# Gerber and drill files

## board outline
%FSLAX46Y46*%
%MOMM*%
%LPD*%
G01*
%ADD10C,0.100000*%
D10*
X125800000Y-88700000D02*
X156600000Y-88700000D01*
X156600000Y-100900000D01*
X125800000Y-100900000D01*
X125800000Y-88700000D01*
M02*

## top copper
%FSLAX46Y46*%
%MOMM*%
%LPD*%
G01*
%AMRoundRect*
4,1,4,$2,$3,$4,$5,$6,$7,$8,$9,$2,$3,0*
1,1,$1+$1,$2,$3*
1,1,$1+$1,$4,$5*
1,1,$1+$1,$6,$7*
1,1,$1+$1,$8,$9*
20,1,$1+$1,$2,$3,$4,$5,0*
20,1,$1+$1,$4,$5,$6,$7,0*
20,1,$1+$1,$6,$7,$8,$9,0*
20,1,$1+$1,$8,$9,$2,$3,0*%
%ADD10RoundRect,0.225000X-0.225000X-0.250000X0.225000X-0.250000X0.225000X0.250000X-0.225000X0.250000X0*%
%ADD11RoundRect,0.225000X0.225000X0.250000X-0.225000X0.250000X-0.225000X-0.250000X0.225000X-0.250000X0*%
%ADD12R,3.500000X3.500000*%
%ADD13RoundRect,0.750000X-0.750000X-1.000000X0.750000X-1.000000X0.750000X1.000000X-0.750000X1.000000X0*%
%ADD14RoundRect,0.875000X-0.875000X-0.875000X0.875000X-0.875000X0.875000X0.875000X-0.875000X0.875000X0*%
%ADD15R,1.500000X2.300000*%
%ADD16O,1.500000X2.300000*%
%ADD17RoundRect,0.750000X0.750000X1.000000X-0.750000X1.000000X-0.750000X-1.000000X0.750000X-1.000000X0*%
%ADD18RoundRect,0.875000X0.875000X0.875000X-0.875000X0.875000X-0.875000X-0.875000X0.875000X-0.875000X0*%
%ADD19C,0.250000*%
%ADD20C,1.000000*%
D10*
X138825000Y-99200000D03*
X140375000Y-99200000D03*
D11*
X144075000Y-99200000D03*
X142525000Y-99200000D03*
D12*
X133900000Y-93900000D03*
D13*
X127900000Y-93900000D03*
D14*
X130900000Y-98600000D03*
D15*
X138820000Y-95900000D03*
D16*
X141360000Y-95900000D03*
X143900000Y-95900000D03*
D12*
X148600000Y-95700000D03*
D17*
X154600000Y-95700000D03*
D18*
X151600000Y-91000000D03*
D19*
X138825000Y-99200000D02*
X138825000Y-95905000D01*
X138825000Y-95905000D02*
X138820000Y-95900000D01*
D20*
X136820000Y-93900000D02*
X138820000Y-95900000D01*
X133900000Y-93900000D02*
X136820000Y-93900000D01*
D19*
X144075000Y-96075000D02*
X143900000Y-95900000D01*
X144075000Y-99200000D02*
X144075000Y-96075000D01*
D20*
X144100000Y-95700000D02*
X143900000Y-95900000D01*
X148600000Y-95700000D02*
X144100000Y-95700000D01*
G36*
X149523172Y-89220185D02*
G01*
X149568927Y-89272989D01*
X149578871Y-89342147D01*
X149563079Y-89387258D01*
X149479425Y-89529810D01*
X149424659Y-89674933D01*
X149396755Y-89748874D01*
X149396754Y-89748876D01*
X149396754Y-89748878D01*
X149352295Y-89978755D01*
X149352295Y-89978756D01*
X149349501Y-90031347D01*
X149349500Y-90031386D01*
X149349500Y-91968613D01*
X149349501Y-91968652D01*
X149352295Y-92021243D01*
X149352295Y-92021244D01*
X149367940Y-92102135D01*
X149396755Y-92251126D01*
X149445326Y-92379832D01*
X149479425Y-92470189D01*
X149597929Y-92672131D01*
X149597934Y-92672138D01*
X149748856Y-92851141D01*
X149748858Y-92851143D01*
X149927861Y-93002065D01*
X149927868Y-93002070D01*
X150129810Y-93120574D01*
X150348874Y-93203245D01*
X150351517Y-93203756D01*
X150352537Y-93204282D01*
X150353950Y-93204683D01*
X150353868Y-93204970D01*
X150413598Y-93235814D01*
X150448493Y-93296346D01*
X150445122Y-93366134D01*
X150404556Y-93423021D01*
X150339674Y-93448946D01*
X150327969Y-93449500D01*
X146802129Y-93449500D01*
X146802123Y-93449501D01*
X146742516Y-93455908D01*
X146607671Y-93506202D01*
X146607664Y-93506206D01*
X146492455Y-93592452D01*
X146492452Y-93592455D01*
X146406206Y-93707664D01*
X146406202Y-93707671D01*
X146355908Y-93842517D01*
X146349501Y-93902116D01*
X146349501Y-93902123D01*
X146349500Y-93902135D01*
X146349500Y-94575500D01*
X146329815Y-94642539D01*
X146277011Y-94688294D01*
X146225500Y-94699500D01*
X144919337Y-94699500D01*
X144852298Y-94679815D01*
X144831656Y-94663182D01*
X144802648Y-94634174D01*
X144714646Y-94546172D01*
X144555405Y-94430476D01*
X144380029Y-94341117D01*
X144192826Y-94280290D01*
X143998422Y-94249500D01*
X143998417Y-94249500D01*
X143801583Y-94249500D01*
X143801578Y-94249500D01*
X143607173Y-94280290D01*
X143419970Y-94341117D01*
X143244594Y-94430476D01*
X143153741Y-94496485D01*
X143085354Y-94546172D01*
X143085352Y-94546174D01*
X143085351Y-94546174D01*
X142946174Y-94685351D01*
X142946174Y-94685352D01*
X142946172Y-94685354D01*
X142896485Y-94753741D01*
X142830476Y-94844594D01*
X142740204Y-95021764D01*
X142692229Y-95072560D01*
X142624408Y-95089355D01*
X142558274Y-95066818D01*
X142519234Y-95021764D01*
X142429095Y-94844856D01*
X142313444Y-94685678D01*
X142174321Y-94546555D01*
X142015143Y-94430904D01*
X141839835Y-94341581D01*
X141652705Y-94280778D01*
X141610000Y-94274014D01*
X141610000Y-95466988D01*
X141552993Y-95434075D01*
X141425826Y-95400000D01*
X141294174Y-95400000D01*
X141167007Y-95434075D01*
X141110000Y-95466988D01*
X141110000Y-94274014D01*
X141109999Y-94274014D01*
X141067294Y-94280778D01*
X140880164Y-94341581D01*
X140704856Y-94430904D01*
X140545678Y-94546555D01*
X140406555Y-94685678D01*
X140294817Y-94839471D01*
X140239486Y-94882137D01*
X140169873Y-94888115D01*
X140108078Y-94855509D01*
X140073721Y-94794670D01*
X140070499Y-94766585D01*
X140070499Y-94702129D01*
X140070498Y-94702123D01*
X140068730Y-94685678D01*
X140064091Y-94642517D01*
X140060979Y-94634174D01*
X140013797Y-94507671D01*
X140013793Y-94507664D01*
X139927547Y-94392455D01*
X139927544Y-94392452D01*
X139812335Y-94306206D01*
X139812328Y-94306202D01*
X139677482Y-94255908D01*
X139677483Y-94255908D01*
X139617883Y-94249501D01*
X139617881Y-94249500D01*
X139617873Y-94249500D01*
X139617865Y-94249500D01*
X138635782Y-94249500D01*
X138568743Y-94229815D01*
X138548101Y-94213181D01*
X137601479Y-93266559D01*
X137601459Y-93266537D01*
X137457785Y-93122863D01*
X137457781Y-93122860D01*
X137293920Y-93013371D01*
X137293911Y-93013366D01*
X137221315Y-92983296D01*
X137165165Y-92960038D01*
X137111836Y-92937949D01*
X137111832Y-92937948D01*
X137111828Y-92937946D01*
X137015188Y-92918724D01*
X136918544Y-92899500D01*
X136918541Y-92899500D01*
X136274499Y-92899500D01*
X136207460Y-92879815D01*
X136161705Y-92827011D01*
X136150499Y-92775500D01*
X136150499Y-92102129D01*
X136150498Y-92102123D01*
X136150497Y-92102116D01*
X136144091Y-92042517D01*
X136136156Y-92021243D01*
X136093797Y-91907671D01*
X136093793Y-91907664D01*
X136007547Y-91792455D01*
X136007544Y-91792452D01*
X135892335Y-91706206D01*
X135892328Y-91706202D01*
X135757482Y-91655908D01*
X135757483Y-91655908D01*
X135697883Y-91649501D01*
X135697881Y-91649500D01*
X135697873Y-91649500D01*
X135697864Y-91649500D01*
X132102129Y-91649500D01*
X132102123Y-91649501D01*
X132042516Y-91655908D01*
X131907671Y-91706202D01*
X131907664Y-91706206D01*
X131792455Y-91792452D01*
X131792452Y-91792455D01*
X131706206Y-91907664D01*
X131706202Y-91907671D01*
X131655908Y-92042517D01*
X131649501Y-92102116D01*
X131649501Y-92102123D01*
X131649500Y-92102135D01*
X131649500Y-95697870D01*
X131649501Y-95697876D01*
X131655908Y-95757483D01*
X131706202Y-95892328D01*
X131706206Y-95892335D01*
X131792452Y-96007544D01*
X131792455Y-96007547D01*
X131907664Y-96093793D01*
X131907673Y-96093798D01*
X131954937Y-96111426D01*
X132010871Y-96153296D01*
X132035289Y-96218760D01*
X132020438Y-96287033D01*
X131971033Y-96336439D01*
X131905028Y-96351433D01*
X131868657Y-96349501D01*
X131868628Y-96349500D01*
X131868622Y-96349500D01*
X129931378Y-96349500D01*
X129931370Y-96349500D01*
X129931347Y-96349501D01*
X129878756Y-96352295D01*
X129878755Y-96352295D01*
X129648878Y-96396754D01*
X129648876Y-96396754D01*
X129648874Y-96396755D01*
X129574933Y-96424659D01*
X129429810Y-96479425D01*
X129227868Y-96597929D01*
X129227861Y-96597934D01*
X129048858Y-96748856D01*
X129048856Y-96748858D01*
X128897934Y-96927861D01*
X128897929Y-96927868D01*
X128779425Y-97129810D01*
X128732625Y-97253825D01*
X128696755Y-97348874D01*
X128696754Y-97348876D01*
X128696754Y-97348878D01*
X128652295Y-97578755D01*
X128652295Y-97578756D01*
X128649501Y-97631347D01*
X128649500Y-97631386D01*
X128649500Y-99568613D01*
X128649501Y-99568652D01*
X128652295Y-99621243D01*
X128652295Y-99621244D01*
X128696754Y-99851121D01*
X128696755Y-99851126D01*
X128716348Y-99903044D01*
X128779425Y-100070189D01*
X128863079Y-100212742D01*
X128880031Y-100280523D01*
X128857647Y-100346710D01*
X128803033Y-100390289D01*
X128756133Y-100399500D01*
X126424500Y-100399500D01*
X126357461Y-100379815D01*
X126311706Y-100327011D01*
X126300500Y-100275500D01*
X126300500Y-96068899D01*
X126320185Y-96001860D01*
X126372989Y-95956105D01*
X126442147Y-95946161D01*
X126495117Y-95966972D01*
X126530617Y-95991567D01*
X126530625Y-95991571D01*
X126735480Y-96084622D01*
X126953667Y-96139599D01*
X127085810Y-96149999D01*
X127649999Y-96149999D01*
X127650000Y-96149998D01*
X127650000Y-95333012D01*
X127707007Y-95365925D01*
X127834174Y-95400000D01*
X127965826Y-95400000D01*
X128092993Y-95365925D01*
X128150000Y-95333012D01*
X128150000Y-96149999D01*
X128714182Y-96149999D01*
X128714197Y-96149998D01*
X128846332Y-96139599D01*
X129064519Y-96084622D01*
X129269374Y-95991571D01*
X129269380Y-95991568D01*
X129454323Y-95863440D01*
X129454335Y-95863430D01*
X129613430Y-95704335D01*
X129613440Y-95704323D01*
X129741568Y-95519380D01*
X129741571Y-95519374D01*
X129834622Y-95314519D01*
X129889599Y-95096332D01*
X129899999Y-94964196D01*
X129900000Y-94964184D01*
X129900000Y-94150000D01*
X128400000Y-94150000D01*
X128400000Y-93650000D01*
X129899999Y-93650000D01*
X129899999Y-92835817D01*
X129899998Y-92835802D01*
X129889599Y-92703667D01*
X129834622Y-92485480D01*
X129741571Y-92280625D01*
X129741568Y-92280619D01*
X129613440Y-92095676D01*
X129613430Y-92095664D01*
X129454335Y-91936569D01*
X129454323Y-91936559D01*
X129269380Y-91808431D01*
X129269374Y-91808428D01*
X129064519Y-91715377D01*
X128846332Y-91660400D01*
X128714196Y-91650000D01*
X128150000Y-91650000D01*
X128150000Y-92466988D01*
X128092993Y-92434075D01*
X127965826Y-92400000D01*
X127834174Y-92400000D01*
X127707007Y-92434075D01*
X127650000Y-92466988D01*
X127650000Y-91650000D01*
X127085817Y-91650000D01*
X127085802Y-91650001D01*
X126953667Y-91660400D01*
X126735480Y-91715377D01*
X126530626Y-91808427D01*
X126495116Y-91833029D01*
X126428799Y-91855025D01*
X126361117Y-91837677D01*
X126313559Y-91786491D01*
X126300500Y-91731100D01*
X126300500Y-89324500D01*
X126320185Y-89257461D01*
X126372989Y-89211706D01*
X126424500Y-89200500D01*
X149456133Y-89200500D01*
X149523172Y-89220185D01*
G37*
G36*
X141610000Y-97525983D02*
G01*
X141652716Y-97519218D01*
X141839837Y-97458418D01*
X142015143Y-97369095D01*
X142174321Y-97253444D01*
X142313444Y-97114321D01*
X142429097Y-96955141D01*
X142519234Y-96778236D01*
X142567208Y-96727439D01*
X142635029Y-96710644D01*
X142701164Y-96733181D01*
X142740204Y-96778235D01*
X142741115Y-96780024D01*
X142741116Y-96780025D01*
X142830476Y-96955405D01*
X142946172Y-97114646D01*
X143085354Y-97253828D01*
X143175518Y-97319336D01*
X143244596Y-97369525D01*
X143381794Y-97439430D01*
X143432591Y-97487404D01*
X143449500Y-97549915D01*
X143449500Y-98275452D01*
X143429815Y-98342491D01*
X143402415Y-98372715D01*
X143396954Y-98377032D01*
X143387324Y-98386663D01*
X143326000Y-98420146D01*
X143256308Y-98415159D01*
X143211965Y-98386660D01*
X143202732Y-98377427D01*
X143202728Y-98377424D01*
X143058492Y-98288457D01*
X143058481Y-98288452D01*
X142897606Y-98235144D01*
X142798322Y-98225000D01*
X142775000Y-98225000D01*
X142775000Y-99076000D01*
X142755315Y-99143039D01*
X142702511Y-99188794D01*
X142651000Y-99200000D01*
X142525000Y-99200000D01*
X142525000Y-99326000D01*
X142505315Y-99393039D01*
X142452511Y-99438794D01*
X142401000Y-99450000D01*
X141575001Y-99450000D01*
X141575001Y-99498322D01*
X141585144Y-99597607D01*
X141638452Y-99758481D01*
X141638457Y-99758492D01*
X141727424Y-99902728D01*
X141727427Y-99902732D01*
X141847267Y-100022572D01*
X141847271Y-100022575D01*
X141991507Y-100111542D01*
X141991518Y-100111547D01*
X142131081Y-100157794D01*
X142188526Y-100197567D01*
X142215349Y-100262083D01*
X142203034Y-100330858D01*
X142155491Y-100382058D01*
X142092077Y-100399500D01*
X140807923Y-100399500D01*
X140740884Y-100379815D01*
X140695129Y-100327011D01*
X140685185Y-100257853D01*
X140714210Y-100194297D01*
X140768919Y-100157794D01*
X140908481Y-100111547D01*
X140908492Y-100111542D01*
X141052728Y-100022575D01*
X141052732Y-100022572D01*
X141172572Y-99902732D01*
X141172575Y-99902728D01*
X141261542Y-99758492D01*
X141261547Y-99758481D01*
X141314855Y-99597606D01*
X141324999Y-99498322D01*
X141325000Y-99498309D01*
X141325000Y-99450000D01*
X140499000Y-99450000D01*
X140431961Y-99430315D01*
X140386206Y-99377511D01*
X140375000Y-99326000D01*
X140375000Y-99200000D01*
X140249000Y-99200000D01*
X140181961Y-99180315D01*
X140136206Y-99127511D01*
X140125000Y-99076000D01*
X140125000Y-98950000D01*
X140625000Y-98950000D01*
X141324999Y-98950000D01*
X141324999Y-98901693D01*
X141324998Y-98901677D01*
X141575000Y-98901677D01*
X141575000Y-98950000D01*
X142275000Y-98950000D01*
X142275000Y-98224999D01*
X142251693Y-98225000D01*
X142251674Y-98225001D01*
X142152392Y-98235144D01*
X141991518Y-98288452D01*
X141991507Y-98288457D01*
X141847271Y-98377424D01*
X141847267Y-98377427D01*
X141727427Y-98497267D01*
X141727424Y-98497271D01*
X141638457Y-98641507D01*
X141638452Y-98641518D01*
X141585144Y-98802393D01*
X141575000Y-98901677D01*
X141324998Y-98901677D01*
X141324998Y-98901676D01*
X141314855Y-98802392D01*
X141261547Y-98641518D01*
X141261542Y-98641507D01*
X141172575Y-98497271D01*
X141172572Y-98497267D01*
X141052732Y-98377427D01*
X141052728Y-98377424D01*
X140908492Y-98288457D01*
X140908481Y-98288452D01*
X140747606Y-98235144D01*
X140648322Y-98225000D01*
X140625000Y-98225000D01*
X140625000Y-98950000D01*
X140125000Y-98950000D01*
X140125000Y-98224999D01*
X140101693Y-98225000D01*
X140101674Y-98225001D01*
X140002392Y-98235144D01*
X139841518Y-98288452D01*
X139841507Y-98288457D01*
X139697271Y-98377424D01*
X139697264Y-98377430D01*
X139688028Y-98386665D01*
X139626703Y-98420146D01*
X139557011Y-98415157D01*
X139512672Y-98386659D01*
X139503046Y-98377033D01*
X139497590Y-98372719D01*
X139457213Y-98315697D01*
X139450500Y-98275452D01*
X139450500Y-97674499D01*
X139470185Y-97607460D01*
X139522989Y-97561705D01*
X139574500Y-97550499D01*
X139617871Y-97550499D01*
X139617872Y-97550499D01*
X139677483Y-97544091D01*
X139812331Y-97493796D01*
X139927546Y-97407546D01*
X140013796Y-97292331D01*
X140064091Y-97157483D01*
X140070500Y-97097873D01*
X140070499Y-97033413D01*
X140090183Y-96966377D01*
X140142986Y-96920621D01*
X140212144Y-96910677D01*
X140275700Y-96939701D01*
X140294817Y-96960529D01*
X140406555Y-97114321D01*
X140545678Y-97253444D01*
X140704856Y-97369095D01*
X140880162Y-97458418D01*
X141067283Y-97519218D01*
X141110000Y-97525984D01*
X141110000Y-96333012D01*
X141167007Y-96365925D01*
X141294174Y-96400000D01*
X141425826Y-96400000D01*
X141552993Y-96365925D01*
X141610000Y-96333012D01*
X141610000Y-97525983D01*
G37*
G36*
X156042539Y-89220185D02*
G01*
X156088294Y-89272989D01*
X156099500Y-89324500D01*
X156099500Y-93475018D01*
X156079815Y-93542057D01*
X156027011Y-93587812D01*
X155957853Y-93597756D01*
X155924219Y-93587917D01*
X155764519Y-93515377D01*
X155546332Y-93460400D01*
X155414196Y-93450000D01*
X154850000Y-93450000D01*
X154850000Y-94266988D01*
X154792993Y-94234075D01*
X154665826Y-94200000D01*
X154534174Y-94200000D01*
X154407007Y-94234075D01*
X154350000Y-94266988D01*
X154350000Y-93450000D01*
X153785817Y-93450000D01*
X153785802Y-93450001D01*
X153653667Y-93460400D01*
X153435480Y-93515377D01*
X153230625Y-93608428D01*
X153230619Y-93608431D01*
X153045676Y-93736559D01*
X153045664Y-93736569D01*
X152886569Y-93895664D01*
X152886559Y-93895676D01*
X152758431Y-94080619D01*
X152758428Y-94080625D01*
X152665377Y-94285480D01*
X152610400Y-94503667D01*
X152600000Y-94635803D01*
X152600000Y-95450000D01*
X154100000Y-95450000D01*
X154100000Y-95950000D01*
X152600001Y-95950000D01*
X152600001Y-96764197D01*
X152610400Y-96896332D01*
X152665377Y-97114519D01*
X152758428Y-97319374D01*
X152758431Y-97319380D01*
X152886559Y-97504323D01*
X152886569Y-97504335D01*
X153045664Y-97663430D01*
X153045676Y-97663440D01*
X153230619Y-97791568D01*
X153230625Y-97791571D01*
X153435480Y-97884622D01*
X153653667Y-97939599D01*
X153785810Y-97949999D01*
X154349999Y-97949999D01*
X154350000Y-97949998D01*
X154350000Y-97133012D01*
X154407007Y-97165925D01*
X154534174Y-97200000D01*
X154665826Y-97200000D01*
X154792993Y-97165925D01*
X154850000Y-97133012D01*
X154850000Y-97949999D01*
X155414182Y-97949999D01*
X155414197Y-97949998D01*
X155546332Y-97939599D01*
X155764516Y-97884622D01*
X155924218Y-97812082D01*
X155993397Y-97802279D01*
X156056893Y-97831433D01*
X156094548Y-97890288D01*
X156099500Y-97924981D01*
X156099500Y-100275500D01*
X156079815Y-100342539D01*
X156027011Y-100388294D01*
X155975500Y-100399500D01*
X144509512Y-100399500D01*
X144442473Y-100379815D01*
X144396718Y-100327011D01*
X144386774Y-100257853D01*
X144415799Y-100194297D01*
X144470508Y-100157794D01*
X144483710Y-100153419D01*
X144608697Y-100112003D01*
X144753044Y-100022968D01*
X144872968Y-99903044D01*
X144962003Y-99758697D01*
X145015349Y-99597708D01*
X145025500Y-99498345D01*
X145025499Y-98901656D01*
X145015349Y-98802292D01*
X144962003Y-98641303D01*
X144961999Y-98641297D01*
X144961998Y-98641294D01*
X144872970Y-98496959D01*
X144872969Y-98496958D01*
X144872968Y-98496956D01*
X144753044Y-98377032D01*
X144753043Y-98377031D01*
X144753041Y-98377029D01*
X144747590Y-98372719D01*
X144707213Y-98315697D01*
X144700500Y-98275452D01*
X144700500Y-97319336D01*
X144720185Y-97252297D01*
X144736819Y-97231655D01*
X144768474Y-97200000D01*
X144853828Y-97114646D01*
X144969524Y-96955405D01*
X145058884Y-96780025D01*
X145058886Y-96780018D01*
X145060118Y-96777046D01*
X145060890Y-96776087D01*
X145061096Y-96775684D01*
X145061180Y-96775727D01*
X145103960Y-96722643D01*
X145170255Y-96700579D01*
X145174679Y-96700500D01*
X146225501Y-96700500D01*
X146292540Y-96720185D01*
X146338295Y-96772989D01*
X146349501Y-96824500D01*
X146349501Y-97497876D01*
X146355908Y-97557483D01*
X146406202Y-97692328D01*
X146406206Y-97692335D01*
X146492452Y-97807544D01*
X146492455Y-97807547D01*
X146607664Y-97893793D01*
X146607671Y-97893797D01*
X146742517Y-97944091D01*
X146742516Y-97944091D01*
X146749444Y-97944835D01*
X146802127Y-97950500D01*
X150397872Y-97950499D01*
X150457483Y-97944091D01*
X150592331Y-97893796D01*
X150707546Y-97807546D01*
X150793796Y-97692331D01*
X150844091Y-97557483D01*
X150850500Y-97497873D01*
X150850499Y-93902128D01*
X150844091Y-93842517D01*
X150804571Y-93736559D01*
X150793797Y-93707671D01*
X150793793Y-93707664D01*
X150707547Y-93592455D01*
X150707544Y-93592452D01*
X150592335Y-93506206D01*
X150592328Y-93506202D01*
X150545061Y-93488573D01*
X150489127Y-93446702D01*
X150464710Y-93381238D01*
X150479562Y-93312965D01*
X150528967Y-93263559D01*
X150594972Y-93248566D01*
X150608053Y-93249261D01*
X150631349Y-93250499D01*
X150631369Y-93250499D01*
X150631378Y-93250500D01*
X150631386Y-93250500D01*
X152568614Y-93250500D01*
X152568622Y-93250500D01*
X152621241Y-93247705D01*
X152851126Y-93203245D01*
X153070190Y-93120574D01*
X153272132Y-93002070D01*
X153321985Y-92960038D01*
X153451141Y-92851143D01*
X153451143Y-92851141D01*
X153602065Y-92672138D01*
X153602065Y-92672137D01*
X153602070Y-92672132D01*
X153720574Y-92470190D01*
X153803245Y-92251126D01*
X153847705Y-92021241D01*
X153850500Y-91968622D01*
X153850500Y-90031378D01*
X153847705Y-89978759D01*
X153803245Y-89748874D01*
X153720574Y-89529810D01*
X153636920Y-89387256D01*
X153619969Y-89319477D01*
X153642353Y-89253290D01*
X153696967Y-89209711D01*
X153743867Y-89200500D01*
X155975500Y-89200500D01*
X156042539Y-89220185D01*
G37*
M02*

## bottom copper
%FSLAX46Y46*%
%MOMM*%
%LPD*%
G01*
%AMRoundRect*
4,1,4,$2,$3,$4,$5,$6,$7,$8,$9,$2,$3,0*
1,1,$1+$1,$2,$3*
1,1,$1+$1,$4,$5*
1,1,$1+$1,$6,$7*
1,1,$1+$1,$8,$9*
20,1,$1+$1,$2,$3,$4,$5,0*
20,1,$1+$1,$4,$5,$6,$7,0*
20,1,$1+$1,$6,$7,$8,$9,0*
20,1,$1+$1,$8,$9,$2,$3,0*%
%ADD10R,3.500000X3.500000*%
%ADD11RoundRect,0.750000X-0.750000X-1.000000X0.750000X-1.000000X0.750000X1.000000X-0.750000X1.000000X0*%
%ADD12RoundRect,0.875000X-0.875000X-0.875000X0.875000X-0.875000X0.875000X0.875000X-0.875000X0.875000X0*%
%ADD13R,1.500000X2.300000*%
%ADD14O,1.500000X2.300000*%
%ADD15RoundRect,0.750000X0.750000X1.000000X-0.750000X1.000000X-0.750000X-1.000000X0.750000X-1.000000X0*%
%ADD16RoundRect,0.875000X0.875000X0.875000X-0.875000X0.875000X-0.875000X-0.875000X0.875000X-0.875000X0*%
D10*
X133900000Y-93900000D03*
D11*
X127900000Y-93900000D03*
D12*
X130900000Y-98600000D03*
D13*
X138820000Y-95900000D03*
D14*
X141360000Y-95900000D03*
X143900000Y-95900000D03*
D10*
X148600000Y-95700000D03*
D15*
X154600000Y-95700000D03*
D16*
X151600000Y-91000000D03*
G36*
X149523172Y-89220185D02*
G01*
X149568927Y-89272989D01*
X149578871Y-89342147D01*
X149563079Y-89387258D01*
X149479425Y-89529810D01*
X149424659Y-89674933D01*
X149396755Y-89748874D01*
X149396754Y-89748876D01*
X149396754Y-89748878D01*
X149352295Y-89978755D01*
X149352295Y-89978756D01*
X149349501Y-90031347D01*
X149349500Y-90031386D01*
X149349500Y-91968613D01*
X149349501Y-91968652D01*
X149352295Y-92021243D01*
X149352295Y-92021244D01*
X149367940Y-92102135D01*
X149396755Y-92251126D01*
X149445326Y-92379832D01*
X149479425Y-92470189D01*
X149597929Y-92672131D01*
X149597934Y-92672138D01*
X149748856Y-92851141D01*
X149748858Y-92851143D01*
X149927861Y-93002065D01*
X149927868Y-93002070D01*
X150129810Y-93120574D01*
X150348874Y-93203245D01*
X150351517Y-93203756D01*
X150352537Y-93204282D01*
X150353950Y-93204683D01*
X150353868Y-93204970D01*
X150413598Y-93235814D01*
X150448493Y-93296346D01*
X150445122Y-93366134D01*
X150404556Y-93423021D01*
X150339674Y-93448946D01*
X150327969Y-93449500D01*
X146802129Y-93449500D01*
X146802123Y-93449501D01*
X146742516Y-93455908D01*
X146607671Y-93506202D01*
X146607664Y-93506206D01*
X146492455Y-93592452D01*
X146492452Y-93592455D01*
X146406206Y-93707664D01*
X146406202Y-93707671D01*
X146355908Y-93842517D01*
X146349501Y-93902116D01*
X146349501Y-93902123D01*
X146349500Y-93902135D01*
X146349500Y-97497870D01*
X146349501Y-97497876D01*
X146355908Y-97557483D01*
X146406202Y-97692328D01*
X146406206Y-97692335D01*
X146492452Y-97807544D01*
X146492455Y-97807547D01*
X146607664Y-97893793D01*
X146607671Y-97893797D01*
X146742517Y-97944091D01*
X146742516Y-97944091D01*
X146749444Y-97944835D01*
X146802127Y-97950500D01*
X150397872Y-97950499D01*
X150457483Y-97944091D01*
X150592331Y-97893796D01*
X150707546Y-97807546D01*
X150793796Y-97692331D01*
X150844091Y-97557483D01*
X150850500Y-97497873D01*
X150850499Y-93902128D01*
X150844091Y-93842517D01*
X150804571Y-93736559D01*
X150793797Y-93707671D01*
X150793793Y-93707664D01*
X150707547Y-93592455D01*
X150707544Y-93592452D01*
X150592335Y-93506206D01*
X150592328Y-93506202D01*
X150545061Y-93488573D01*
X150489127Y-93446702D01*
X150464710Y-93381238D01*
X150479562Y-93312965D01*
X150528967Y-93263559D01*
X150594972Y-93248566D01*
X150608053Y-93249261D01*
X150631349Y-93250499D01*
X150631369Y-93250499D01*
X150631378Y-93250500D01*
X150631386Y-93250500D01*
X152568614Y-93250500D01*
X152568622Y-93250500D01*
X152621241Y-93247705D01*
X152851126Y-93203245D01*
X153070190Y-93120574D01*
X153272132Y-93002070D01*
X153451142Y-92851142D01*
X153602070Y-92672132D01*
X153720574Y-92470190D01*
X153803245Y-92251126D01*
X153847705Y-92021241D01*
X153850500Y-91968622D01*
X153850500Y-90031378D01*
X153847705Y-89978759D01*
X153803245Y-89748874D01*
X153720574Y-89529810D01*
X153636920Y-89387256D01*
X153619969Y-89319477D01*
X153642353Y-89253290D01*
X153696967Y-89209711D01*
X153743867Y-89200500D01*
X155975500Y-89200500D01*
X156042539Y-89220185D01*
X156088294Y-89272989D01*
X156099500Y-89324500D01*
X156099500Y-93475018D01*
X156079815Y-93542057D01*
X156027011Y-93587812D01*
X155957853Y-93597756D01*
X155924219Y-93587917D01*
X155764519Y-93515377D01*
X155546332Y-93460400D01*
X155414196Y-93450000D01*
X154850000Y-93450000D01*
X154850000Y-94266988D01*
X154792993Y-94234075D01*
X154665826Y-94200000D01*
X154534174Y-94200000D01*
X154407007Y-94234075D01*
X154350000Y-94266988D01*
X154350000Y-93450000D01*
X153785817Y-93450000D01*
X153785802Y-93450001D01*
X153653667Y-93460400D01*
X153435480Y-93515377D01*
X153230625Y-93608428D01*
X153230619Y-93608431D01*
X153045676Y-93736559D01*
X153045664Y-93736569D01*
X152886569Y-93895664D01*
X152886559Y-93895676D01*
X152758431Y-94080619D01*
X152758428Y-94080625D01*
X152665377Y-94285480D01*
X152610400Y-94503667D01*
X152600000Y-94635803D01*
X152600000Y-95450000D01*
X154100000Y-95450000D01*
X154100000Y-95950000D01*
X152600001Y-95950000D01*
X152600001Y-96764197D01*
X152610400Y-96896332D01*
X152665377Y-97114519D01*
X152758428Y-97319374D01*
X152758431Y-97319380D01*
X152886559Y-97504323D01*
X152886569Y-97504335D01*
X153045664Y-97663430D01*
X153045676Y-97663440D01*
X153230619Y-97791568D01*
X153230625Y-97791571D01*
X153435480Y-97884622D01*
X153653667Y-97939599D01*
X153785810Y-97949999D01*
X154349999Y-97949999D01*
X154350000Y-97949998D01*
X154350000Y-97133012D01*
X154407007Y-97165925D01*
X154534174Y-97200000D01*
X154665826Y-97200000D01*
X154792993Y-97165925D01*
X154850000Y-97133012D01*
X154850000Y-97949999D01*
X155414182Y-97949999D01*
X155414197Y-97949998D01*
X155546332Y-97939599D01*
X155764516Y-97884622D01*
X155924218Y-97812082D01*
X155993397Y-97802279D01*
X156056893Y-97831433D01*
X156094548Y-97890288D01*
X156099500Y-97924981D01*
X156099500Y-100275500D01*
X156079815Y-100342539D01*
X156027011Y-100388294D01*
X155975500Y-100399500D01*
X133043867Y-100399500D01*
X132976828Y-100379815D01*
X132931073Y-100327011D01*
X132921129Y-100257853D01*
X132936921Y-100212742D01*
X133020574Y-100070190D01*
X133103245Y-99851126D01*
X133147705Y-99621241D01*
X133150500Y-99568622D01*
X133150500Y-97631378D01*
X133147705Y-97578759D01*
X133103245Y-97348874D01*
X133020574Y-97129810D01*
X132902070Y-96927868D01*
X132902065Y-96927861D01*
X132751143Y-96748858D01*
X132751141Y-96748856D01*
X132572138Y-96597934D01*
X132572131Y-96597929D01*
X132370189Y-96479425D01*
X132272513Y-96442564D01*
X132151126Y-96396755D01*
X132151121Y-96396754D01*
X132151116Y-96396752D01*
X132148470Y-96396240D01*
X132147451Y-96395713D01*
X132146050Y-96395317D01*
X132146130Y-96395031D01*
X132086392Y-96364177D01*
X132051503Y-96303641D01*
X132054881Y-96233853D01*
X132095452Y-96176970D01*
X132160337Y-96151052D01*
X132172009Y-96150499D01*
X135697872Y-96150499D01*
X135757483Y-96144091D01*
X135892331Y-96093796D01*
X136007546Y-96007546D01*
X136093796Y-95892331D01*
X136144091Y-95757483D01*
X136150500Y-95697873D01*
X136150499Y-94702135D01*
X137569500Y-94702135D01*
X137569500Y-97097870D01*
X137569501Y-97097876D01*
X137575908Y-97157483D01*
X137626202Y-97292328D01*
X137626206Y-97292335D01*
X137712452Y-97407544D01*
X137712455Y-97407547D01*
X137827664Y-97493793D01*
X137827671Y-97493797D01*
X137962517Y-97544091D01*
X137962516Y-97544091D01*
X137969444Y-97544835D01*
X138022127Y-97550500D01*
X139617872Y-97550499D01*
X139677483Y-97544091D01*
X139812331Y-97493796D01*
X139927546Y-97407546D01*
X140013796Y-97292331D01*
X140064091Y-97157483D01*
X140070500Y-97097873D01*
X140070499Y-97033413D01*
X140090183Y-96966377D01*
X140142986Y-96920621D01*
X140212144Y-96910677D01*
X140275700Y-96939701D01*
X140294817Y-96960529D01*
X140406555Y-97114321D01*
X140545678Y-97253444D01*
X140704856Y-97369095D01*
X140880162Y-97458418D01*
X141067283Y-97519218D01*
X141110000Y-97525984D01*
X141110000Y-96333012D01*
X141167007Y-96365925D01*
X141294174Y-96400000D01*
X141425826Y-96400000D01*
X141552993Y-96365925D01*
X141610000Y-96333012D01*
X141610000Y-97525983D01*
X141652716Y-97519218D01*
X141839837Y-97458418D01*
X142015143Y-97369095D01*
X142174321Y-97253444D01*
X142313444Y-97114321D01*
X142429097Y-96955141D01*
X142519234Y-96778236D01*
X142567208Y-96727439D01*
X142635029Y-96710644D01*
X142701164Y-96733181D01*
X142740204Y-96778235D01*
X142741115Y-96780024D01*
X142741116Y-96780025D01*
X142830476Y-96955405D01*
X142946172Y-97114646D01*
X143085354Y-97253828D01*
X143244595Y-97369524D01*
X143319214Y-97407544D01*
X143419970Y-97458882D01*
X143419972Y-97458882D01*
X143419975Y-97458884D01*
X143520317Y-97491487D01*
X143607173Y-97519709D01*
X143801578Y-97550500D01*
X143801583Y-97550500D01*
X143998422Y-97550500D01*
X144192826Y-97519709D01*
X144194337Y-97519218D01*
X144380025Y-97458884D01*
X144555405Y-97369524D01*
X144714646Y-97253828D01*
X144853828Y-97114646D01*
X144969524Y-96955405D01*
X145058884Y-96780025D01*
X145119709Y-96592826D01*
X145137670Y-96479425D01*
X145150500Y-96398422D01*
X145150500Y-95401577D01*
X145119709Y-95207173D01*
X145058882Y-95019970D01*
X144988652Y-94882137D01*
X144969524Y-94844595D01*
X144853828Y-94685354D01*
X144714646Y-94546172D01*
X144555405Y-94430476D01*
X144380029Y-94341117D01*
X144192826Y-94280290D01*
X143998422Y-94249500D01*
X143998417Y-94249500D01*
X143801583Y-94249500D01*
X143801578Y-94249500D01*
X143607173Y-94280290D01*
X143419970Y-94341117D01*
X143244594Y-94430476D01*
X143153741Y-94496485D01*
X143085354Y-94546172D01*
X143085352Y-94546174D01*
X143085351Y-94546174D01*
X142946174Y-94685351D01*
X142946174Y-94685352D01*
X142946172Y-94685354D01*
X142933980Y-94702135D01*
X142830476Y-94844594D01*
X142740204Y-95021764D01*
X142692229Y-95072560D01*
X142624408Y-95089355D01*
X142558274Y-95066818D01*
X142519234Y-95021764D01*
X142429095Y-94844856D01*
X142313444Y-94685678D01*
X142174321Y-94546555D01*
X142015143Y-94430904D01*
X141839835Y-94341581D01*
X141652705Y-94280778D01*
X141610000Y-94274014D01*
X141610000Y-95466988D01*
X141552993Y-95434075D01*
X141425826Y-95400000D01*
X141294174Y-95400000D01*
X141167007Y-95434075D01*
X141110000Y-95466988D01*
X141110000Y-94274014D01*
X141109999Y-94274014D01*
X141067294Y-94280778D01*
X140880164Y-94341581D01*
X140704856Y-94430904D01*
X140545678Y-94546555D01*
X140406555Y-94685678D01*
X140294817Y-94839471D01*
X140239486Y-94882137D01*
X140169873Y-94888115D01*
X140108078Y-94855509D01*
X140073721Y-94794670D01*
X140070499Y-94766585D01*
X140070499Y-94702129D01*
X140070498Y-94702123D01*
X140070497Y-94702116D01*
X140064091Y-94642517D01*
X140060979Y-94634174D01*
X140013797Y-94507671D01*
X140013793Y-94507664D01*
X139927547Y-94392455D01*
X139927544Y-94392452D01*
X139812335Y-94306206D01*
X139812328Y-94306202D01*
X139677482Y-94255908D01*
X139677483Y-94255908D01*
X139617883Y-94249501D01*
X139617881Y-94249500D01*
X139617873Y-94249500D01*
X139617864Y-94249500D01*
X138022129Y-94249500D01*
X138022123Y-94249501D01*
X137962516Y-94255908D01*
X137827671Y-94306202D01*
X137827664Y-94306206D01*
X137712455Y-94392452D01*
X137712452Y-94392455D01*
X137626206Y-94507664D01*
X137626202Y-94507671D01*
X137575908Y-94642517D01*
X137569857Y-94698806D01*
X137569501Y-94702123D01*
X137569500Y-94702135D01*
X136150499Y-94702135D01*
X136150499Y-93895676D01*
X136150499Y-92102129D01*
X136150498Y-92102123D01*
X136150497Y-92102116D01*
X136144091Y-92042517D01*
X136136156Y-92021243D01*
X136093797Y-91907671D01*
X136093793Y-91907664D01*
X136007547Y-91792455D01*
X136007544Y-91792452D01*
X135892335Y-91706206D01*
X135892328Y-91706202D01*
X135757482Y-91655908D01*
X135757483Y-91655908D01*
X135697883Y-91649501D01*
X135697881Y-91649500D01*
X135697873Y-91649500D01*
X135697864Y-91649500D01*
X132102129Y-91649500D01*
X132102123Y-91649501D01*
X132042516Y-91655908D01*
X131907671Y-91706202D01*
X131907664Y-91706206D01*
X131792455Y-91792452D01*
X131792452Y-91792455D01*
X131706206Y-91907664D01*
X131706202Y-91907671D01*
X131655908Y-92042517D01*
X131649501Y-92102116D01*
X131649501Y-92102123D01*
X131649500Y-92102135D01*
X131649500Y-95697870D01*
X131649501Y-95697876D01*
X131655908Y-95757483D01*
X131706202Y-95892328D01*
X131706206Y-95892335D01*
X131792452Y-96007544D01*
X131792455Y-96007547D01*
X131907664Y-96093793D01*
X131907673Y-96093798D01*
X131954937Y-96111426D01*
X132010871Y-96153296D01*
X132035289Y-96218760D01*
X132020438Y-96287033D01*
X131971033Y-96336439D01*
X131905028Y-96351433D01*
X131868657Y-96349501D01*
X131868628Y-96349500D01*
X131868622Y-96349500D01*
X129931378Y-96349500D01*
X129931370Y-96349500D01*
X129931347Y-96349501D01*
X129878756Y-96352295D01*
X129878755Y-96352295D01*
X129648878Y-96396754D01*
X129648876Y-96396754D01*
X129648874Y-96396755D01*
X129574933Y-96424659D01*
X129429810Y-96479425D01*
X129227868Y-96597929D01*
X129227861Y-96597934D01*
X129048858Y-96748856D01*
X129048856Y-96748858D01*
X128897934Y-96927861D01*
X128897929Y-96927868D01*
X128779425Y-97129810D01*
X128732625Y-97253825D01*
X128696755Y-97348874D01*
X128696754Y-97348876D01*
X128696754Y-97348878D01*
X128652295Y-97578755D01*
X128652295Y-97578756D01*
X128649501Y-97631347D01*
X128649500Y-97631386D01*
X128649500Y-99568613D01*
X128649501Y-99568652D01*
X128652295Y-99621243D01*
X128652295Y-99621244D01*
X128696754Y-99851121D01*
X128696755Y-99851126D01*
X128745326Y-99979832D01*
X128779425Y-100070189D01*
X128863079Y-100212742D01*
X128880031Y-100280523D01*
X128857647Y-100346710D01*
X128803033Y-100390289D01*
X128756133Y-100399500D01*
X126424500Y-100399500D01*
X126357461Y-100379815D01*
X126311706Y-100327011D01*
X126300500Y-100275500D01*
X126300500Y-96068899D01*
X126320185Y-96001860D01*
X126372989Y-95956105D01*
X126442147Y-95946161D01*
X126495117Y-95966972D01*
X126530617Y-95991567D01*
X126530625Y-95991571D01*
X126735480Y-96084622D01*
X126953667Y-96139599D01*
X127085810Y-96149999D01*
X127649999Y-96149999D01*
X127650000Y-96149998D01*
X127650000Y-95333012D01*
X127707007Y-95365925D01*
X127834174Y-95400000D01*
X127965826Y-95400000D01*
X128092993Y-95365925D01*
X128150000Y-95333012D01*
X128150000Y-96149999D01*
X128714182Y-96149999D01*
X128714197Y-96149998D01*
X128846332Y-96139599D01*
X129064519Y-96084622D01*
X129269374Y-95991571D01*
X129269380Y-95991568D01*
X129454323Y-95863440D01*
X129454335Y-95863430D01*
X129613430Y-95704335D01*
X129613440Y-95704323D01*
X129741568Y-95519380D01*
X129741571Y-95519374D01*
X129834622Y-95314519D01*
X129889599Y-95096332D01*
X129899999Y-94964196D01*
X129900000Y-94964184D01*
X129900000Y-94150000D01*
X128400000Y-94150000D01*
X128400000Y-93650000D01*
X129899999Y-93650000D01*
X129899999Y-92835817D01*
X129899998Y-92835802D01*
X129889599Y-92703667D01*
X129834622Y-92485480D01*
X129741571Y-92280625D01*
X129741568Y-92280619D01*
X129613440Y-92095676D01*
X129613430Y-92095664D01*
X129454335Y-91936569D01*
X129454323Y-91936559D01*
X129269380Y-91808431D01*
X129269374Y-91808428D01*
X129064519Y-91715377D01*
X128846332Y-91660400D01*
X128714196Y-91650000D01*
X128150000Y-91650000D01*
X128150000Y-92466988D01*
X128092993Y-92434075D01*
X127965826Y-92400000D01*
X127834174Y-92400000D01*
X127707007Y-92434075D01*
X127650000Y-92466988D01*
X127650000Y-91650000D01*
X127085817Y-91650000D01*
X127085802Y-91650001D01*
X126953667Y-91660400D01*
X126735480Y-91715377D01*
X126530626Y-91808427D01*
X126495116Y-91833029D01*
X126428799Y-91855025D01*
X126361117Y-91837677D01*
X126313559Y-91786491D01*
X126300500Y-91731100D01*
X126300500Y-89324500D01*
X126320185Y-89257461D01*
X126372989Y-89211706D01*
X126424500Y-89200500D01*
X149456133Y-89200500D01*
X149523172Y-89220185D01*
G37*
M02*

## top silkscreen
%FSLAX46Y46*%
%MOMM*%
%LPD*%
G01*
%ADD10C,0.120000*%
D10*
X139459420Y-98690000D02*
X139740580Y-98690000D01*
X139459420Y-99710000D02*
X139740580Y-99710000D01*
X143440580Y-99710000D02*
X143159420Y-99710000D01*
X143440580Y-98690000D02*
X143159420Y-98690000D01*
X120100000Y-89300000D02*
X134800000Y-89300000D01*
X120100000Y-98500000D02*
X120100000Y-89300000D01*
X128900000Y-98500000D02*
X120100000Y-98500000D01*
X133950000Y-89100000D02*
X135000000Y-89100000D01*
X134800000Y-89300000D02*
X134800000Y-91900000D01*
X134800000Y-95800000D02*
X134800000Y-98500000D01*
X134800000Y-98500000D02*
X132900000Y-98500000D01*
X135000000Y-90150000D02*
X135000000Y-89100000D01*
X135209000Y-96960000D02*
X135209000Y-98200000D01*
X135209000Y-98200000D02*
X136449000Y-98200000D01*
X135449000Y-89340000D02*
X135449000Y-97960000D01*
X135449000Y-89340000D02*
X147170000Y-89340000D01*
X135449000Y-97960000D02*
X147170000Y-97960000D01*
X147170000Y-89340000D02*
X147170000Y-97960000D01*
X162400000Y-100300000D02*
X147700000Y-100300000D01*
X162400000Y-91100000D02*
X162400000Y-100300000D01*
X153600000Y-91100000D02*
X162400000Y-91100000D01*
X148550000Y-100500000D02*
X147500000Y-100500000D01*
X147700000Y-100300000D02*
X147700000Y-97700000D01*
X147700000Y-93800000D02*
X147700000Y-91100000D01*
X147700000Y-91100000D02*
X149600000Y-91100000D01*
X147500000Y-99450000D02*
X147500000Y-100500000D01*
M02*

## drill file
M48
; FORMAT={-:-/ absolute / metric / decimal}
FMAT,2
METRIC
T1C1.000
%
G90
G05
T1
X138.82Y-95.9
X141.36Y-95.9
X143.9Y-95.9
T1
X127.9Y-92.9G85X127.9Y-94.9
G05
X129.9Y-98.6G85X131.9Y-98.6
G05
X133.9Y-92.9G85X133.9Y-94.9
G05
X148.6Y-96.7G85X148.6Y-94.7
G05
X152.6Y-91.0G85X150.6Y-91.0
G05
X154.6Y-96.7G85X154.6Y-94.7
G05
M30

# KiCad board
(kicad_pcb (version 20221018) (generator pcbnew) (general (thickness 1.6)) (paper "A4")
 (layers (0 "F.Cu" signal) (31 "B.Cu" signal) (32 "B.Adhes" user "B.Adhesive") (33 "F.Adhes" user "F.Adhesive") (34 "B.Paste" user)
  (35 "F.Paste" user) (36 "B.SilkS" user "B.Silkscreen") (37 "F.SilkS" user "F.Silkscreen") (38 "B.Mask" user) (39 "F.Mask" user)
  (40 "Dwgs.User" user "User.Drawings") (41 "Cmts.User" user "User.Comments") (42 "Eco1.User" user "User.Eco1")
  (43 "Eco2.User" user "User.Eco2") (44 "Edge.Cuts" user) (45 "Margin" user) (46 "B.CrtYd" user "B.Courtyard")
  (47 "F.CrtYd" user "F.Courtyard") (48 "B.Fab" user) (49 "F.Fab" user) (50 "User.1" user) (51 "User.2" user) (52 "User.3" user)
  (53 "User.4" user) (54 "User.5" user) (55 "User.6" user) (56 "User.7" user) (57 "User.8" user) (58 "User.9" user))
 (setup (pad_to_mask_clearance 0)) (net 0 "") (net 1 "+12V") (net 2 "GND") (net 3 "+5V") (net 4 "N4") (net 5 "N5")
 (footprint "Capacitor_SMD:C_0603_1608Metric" (layer "F.Cu") (at 139.6 99.2)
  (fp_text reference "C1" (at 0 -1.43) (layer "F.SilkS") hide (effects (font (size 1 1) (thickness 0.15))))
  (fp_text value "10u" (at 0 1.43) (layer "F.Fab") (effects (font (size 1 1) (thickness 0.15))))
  (fp_line (start -0.14058 -0.51) (end 0.14058 -0.51) (stroke (width 0.12) (type solid)) (layer "F.SilkS"))
  (fp_line (start -0.14058 0.51) (end 0.14058 0.51) (stroke (width 0.12) (type solid)) (layer "F.SilkS"))
  (pad "1" smd roundrect (at -0.775 0) (size 0.9 0.95) (layers "F.Cu" "F.Paste" "F.Mask") (roundrect_rratio 0.25) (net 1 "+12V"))
  (pad "2" smd roundrect (at 0.775 0) (size 0.9 0.95) (layers "F.Cu" "F.Paste" "F.Mask") (roundrect_rratio 0.25) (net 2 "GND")))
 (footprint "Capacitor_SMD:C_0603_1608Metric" (layer "F.Cu") (at 143.3 99.2 180)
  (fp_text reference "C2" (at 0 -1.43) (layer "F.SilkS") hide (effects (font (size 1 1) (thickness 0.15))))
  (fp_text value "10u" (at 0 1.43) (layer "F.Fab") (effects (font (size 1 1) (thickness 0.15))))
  (fp_line (start -0.14058 -0.51) (end 0.14058 -0.51) (stroke (width 0.12) (type solid)) (layer "F.SilkS"))
  (fp_line (start -0.14058 0.51) (end 0.14058 0.51) (stroke (width 0.12) (type solid)) (layer "F.SilkS"))
  (pad "1" smd roundrect (at -0.775 0 180) (size 0.9 0.95) (layers "F.Cu" "F.Paste" "F.Mask") (roundrect_rratio 0.25) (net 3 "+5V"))
  (pad "2" smd roundrect (at 0.775 0 180) (size 0.9 0.95) (layers "F.Cu" "F.Paste" "F.Mask") (roundrect_rratio 0.25) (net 2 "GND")))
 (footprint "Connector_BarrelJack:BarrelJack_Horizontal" (layer "F.Cu") (at 133.9 93.9)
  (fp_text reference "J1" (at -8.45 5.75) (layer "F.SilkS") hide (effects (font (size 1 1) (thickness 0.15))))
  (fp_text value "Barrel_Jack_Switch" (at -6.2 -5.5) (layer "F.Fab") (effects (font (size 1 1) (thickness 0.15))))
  (fp_line (start -13.8 -4.6) (end 0.9 -4.6) (stroke (width 0.12) (type solid)) (layer "F.SilkS"))
  (fp_line (start -13.8 4.6) (end -13.8 -4.6) (stroke (width 0.12) (type solid)) (layer "F.SilkS"))
  (fp_line (start -5 4.6) (end -13.8 4.6) (stroke (width 0.12) (type solid)) (layer "F.SilkS"))
  (fp_line (start 0.05 -4.8) (end 1.1 -4.8) (stroke (width 0.12) (type solid)) (layer "F.SilkS"))
  (fp_line (start 0.9 -4.6) (end 0.9 -2) (stroke (width 0.12) (type solid)) (layer "F.SilkS"))
  (fp_line (start 0.9 1.9) (end 0.9 4.6) (stroke (width 0.12) (type solid)) (layer "F.SilkS"))
  (fp_line (start 0.9 4.6) (end -1 4.6) (stroke (width 0.12) (type solid)) (layer "F.SilkS"))
  (fp_line (start 1.1 -3.75) (end 1.1 -4.8) (stroke (width 0.12) (type solid)) (layer "F.SilkS"))
  (pad "1" thru_hole rect (at 0 0) (size 3.5 3.5) (drill oval 1 3) (layers "*.Cu" "*.Mask") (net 1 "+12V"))
  (pad "2" thru_hole roundrect (at -6 0) (size 3 3.5) (drill oval 1 3) (layers "*.Cu" "*.Mask") (roundrect_rratio 0.25) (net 2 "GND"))
  (pad "3" thru_hole roundrect (at -3 4.7) (size 3.5 3.5) (drill oval 3 1) (layers "*.Cu" "*.Mask") (roundrect_rratio 0.25) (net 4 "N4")))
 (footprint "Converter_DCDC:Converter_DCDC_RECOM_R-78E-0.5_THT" (layer "F.Cu") (at 138.82 95.9)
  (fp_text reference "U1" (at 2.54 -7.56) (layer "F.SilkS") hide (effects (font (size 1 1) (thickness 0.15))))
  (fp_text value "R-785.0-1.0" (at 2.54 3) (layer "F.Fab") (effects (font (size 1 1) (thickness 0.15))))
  (fp_line (start -3.611 1.06) (end -3.611 2.3) (stroke (width 0.12) (type solid)) (layer "F.SilkS"))
  (fp_line (start -3.611 2.3) (end -2.371 2.3) (stroke (width 0.12) (type solid)) (layer "F.SilkS"))
  (fp_line (start -3.371 -6.56) (end -3.371 2.06) (stroke (width 0.12) (type solid)) (layer "F.SilkS"))
  (fp_line (start -3.371 -6.56) (end 8.35 -6.56) (stroke (width 0.12) (type solid)) (layer "F.SilkS"))
  (fp_line (start -3.371 2.06) (end 8.35 2.06) (stroke (width 0.12) (type solid)) (layer "F.SilkS"))
  (fp_line (start 8.35 -6.56) (end 8.35 2.06) (stroke (width 0.12) (type solid)) (layer "F.SilkS"))
  (pad "1" thru_hole rect (at 0 0) (size 1.5 2.3) (drill 1) (layers "*.Cu" "*.Mask") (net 1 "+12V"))
  (pad "2" thru_hole oval (at 2.54 0) (size 1.5 2.3) (drill 1) (layers "*.Cu" "*.Mask") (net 2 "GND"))
  (pad "3" thru_hole oval (at 5.08 0) (size 1.5 2.3) (drill 1) (layers "*.Cu" "*.Mask") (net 3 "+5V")))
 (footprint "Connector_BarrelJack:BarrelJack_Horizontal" (layer "F.Cu") (at 148.6 95.7 180)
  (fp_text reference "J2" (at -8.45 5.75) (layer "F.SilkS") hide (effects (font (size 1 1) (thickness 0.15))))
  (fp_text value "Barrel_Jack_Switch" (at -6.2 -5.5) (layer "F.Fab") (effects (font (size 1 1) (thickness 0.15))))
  (fp_line (start -13.8 -4.6) (end 0.9 -4.6) (stroke (width 0.12) (type solid)) (layer "F.SilkS"))
  (fp_line (start -13.8 4.6) (end -13.8 -4.6) (stroke (width 0.12) (type solid)) (layer "F.SilkS"))
  (fp_line (start -5 4.6) (end -13.8 4.6) (stroke (width 0.12) (type solid)) (layer "F.SilkS"))
  (fp_line (start 0.05 -4.8) (end 1.1 -4.8) (stroke (width 0.12) (type solid)) (layer "F.SilkS"))
  (fp_line (start 0.9 -4.6) (end 0.9 -2) (stroke (width 0.12) (type solid)) (layer "F.SilkS"))
  (fp_line (start 0.9 1.9) (end 0.9 4.6) (stroke (width 0.12) (type solid)) (layer "F.SilkS"))
  (fp_line (start 0.9 4.6) (end -1 4.6) (stroke (width 0.12) (type solid)) (layer "F.SilkS"))
  (fp_line (start 1.1 -3.75) (end 1.1 -4.8) (stroke (width 0.12) (type solid)) (layer "F.SilkS"))
  (pad "1" thru_hole rect (at 0 0 180) (size 3.5 3.5) (drill oval 1 3) (layers "*.Cu" "*.Mask") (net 3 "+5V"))
  (pad "2" thru_hole roundrect (at -6 0 180) (size 3 3.5) (drill oval 1 3) (layers "*.Cu" "*.Mask") (roundrect_rratio 0.25) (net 2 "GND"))
  (pad "3" thru_hole roundrect (at -3 4.7 180) (size 3.5 3.5) (drill oval 3 1) (layers "*.Cu" "*.Mask") (roundrect_rratio 0.25) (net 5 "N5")))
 (gr_rect (start 125.8 88.7) (end 156.6 100.9) (stroke (width 0.1) (type default)) (fill none) (layer "Edge.Cuts"))
 (segment (start 138.825 99.2) (end 138.825 95.905) (width 0.25) (layer "F.Cu") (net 1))
 (segment (start 138.825 95.905) (end 138.82 95.9) (width 0.25) (layer "F.Cu") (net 1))
 (segment (start 136.82 93.9) (end 138.82 95.9) (width 1) (layer "F.Cu") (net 1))
 (segment (start 133.9 93.9) (end 136.82 93.9) (width 1) (layer "F.Cu") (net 1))
 (segment (start 144.075 96.075) (end 143.9 95.9) (width 0.25) (layer "F.Cu") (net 3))
 (segment (start 144.075 99.2) (end 144.075 96.075) (width 0.25) (layer "F.Cu") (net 3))
 (segment (start 144.1 95.7) (end 143.9 95.9) (width 1) (layer "F.Cu") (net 3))
 (segment (start 148.6 95.7) (end 144.1 95.7) (width 1) (layer "F.Cu") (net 3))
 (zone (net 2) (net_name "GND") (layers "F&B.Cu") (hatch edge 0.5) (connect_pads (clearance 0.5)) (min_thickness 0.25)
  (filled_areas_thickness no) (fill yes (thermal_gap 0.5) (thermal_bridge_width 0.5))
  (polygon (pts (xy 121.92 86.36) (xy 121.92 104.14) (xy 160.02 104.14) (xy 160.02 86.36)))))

